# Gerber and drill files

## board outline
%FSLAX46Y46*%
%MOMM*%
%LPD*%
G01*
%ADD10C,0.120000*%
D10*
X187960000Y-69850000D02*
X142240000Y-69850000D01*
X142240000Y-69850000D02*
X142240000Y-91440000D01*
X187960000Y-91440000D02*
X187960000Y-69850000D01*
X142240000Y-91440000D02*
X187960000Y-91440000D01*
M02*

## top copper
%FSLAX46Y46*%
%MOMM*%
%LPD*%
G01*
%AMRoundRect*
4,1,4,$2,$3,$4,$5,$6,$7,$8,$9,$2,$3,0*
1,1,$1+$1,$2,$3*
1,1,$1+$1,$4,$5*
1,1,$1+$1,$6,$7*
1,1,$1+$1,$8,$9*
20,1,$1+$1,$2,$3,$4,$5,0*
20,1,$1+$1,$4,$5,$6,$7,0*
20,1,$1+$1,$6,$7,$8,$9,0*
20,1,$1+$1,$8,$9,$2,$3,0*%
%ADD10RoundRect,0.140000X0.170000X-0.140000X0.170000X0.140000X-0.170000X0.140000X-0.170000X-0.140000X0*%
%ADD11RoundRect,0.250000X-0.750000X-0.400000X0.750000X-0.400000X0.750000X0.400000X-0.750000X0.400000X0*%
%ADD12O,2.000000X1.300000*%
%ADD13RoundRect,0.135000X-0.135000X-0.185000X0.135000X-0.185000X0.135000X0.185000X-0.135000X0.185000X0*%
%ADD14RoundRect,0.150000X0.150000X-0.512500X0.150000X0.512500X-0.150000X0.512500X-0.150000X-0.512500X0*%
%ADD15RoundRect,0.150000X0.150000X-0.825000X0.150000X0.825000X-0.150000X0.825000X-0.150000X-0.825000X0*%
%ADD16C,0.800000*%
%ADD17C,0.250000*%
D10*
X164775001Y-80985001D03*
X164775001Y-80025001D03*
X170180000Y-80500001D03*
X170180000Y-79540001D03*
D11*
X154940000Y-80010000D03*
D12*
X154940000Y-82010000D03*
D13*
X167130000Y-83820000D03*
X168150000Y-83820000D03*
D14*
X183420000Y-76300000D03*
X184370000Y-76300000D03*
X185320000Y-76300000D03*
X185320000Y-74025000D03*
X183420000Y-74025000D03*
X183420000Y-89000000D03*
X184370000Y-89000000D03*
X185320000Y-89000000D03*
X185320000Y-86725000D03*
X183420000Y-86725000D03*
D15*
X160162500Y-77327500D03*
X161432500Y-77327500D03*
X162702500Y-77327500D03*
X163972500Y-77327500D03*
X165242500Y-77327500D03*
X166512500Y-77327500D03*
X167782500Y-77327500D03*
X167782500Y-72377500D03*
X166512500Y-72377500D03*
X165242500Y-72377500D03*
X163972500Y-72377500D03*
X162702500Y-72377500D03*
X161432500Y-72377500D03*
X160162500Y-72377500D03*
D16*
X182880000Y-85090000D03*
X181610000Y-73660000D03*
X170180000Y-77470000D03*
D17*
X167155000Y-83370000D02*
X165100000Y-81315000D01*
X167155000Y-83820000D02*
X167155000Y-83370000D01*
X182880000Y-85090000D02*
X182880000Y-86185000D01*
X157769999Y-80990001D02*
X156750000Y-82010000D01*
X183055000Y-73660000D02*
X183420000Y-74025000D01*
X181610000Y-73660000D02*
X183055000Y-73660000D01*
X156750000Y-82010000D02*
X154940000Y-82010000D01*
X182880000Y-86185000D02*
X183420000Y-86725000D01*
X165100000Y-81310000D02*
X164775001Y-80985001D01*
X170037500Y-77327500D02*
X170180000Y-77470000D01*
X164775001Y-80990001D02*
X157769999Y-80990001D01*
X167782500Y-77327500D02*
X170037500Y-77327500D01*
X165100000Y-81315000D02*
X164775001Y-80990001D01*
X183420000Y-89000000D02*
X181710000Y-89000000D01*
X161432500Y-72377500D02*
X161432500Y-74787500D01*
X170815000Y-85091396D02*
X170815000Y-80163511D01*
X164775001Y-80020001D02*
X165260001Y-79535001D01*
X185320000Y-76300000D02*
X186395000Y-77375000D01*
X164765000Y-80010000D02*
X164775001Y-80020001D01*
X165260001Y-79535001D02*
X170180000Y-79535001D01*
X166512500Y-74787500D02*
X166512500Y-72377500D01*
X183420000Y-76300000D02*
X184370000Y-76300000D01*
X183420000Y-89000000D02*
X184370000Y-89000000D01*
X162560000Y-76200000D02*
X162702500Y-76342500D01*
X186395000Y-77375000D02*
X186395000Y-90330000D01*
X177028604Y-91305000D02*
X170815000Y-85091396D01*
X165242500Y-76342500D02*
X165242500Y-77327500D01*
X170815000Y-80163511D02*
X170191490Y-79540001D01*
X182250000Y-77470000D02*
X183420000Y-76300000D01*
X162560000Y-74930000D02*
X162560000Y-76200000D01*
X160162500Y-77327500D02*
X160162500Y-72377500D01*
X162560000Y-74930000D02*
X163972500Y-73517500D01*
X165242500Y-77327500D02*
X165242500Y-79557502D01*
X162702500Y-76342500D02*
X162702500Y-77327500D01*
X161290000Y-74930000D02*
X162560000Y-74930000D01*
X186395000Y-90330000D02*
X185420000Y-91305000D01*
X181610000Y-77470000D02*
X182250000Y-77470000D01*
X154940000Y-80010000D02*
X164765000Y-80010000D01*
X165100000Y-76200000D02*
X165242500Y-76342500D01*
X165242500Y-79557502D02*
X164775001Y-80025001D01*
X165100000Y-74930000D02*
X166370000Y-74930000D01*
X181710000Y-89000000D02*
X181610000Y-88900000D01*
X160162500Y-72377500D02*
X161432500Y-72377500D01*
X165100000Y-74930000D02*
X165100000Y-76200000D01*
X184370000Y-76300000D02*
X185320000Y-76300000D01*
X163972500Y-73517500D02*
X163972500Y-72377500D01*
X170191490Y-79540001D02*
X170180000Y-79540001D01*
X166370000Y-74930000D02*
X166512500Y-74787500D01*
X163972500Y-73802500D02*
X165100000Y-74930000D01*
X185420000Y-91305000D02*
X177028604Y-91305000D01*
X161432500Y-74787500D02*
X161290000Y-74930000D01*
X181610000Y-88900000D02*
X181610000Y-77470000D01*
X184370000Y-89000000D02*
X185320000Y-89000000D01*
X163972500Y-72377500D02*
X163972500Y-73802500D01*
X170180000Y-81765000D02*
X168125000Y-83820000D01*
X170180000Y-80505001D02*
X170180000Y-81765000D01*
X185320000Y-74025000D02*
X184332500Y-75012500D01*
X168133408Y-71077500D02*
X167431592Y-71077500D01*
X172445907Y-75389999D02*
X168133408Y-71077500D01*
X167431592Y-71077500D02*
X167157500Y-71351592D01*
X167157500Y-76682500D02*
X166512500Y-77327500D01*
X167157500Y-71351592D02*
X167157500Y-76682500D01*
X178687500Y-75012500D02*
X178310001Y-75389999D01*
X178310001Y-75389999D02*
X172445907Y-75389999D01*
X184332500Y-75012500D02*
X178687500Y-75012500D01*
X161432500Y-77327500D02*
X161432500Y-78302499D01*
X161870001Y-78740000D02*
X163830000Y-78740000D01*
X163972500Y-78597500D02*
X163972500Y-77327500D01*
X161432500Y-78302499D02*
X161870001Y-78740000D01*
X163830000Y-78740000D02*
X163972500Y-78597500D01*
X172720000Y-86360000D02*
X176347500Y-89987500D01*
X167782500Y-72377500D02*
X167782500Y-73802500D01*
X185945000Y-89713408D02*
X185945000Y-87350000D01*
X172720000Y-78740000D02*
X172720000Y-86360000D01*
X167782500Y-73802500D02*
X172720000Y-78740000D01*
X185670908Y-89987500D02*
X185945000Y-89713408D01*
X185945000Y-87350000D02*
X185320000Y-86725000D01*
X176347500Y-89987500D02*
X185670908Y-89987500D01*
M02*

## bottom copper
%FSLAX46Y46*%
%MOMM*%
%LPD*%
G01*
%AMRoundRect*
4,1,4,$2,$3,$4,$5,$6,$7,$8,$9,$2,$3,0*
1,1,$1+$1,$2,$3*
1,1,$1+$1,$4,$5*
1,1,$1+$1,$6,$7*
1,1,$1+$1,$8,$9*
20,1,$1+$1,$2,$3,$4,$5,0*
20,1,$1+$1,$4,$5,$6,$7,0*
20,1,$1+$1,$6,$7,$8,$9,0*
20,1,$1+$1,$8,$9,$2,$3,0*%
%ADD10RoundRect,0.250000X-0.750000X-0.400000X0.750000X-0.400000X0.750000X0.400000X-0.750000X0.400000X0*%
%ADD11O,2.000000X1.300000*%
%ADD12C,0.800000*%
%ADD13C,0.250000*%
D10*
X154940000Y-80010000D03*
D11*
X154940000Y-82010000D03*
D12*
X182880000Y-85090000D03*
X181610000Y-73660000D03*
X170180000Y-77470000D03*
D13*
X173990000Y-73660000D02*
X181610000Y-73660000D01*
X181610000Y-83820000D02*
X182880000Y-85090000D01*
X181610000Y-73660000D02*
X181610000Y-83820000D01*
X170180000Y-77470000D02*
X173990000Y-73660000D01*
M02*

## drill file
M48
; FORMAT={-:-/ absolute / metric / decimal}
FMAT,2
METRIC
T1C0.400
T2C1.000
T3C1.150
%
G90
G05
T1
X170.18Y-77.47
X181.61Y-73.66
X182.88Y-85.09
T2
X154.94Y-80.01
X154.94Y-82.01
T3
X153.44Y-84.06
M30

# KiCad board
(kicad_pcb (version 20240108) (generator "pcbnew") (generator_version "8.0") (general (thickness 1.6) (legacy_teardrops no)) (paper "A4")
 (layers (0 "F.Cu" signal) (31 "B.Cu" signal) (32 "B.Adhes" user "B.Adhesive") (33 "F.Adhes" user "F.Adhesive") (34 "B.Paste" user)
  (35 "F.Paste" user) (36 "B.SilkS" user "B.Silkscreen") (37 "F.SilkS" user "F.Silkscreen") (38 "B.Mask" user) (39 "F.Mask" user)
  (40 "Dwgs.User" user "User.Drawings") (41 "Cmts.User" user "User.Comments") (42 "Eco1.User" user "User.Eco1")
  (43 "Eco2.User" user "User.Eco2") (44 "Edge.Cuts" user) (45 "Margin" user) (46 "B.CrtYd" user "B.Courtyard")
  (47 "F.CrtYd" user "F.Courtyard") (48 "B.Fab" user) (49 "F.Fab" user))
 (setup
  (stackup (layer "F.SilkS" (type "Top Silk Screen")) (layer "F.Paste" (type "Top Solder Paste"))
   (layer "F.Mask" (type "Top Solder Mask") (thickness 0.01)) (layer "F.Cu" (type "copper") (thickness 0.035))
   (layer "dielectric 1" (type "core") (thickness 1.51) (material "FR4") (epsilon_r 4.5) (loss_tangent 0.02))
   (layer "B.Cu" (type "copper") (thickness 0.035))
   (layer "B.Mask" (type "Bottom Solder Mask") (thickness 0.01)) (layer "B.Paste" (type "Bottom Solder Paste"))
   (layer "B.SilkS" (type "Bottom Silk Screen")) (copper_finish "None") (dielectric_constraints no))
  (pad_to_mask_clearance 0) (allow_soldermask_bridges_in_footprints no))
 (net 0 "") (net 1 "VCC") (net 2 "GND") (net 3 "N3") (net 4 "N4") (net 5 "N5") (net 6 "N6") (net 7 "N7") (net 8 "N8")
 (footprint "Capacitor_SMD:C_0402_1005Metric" (layer "F.Cu") (at 164.775001 80.505001 90)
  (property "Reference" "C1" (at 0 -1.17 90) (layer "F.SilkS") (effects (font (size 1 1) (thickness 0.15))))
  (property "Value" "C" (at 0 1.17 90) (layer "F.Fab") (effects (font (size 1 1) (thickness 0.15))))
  (pad "1" smd roundrect (at -0.48 0 90) (size 0.56 0.62) (layers "F.Cu" "F.Paste" "F.Mask") (roundrect_rratio 0.25) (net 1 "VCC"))
  (pad "2" smd roundrect (at 0.48 0 90) (size 0.56 0.62) (layers "F.Cu" "F.Paste" "F.Mask") (roundrect_rratio 0.25) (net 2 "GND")))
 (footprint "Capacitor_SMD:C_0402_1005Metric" (layer "F.Cu") (at 170.18 80.020001 90)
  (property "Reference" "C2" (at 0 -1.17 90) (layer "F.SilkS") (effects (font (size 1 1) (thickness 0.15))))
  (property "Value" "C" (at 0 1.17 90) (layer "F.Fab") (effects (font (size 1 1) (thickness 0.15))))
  (pad "1" smd roundrect (at -0.48 0 90) (size 0.56 0.62) (layers "F.Cu" "F.Paste" "F.Mask") (roundrect_rratio 0.25) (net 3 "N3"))
  (pad "2" smd roundrect (at 0.48 0 90) (size 0.56 0.62) (layers "F.Cu" "F.Paste" "F.Mask") (roundrect_rratio 0.25) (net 2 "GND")))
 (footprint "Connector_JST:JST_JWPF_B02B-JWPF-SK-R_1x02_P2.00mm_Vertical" (layer "F.Cu") (at 154.94 80.01)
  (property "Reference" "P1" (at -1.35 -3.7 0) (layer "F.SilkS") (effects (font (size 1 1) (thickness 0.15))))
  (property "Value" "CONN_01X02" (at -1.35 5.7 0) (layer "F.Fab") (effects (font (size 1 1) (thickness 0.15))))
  (pad "" np_thru_hole circle (at -1.5 4.05) (size 1.15 1.15) (drill 1.15) (layers "*.Cu" "*.Mask"))
  (pad "1" thru_hole roundrect (at 0 0) (size 2 1.3) (drill 1) (layers "*.Cu" "*.Mask") (remove_unused_layers no)
   (roundrect_rratio 0.192308) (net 2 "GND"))
  (pad "2" thru_hole oval (at 0 2) (size 2 1.3) (drill 1) (layers "*.Cu" "*.Mask") (remove_unused_layers no) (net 1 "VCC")))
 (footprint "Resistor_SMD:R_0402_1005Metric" (layer "F.Cu") (at 167.64 83.82)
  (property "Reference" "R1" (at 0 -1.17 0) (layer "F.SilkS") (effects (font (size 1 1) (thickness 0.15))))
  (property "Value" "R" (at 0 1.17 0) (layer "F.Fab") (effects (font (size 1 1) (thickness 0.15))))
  (pad "1" smd roundrect (at -0.51 0) (size 0.54 0.64) (layers "F.Cu" "F.Paste" "F.Mask") (roundrect_rratio 0.25) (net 1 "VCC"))
  (pad "2" smd roundrect (at 0.51 0) (size 0.54 0.64) (layers "F.Cu" "F.Paste" "F.Mask") (roundrect_rratio 0.25) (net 3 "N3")))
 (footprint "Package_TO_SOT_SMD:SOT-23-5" (layer "F.Cu") (at 184.37 75.1625 90)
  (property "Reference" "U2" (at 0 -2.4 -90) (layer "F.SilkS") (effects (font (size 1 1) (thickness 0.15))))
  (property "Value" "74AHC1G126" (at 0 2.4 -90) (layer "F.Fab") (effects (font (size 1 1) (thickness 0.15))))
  (pad "1" smd roundrect (at -1.1375 -0.95 90) (size 1.325 0.6) (layers "F.Cu" "F.Paste" "F.Mask") (roundrect_rratio 0.25) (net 2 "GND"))
  (pad "2" smd roundrect (at -1.1375 0 90) (size 1.325 0.6) (layers "F.Cu" "F.Paste" "F.Mask") (roundrect_rratio 0.25) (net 2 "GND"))
  (pad "3" smd roundrect (at -1.1375 0.95 90) (size 1.325 0.6) (layers "F.Cu" "F.Paste" "F.Mask") (roundrect_rratio 0.25) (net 2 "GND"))
  (pad "4" smd roundrect (at 1.1375 0.95 90) (size 1.325 0.6) (layers "F.Cu" "F.Paste" "F.Mask") (roundrect_rratio 0.25) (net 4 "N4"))
  (pad "5" smd roundrect (at 1.1375 -0.95 90) (size 1.325 0.6) (layers "F.Cu" "F.Paste" "F.Mask") (roundrect_rratio 0.25) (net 1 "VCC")))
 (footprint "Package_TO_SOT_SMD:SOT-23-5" (layer "F.Cu") (at 184.37 87.8625 90)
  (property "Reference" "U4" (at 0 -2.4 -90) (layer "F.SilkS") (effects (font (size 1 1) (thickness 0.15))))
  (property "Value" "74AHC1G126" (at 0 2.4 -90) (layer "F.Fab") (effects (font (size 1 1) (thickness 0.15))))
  (pad "1" smd roundrect (at -1.1375 -0.95 90) (size 1.325 0.6) (layers "F.Cu" "F.Paste" "F.Mask") (roundrect_rratio 0.25) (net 2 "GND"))
  (pad "2" smd roundrect (at -1.1375 0 90) (size 1.325 0.6) (layers "F.Cu" "F.Paste" "F.Mask") (roundrect_rratio 0.25) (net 2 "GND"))
  (pad "3" smd roundrect (at -1.1375 0.95 90) (size 1.325 0.6) (layers "F.Cu" "F.Paste" "F.Mask") (roundrect_rratio 0.25) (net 2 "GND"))
  (pad "4" smd roundrect (at 1.1375 0.95 90) (size 1.325 0.6) (layers "F.Cu" "F.Paste" "F.Mask") (roundrect_rratio 0.25) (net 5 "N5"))
  (pad "5" smd roundrect (at 1.1375 -0.95 90) (size 1.325 0.6) (layers "F.Cu" "F.Paste" "F.Mask") (roundrect_rratio 0.25) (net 1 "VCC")))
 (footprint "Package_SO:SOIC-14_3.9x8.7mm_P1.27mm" (layer "F.Cu") (at 163.9725 74.8525 90)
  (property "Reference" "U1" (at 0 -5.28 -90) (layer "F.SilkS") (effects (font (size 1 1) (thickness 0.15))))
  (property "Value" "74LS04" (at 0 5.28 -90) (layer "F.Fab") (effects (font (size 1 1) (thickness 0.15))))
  (pad "1" smd roundrect (at -2.475 -3.81 90) (size 1.95 0.6) (layers "F.Cu" "F.Paste" "F.Mask") (roundrect_rratio 0.25) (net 2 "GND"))
  (pad "2" smd roundrect (at -2.475 -2.54 90) (size 1.95 0.6) (layers "F.Cu" "F.Paste" "F.Mask") (roundrect_rratio 0.25) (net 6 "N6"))
  (pad "3" smd roundrect (at -2.475 -1.27 90) (size 1.95 0.6) (layers "F.Cu" "F.Paste" "F.Mask") (roundrect_rratio 0.25) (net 2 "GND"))
  (pad "4" smd roundrect (at -2.475 0 90) (size 1.95 0.6) (layers "F.Cu" "F.Paste" "F.Mask") (roundrect_rratio 0.25) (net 6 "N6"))
  (pad "5" smd roundrect (at -2.475 1.27 90) (size 1.95 0.6) (layers "F.Cu" "F.Paste" "F.Mask") (roundrect_rratio 0.25) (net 2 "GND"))
  (pad "6" smd roundrect (at -2.475 2.54 90) (size 1.95 0.6) (layers "F.Cu" "F.Paste" "F.Mask") (roundrect_rratio 0.25) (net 4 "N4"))
  (pad "7" smd roundrect (at -2.475 3.81 90) (size 1.95 0.6) (layers "F.Cu" "F.Paste" "F.Mask") (roundrect_rratio 0.25) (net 1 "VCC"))
  (pad "8" smd roundrect (at 2.475 3.81 90) (size 1.95 0.6) (layers "F.Cu" "F.Paste" "F.Mask") (roundrect_rratio 0.25) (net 5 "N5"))
  (pad "9" smd roundrect (at 2.475 2.54 90) (size 1.95 0.6) (layers "F.Cu" "F.Paste" "F.Mask") (roundrect_rratio 0.25) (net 2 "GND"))
  (pad "10" smd roundrect (at 2.475 1.27 90) (size 1.95 0.6) (layers "F.Cu" "F.Paste" "F.Mask") (roundrect_rratio 0.25) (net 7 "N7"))
  (pad "11" smd roundrect (at 2.475 0 90) (size 1.95 0.6) (layers "F.Cu" "F.Paste" "F.Mask") (roundrect_rratio 0.25) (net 2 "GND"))
  (pad "12" smd roundrect (at 2.475 -1.27 90) (size 1.95 0.6) (layers "F.Cu" "F.Paste" "F.Mask") (roundrect_rratio 0.25) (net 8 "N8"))
  (pad "13" smd roundrect (at 2.475 -2.54 90) (size 1.95 0.6) (layers "F.Cu" "F.Paste" "F.Mask") (roundrect_rratio 0.25) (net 2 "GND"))
  (pad "14" smd roundrect (at 2.475 -3.81 90) (size 1.95 0.6) (layers "F.Cu" "F.Paste" "F.Mask") (roundrect_rratio 0.25) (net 2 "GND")))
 (gr_line (start 187.96 69.85) (end 142.24 69.85) (stroke (width 0.12) (type solid)) (layer "Edge.Cuts"))
 (gr_line (start 142.24 69.85) (end 142.24 91.44) (stroke (width 0.12) (type solid)) (layer "Edge.Cuts"))
 (gr_line (start 187.96 91.44) (end 187.96 69.85) (stroke (width 0.12) (type solid)) (layer "Edge.Cuts"))
 (gr_line (start 142.24 91.44) (end 187.96 91.44) (stroke (width 0.12) (type solid)) (layer "Edge.Cuts"))
 (segment (start 167.155 83.37) (end 165.1 81.315) (width 0.25) (layer "F.Cu") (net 1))
 (segment (start 167.155 83.82) (end 167.155 83.37) (width 0.25) (layer "F.Cu") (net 1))
 (segment (start 182.88 85.09) (end 182.88 86.185) (width 0.25) (layer "F.Cu") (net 1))
 (segment (start 157.769999 80.990001) (end 156.75 82.01) (width 0.25) (layer "F.Cu") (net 1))
 (segment (start 183.055 73.66) (end 183.42 74.025) (width 0.25) (layer "F.Cu") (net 1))
 (segment (start 181.61 73.66) (end 183.055 73.66) (width 0.25) (layer "F.Cu") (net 1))
 (segment (start 156.75 82.01) (end 154.94 82.01) (width 0.25) (layer "F.Cu") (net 1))
 (segment (start 182.88 86.185) (end 183.42 86.725) (width 0.25) (layer "F.Cu") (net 1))
 (segment (start 165.1 81.31) (end 164.775001 80.985001) (width 0.25) (layer "F.Cu") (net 1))
 (segment (start 170.0375 77.3275) (end 170.18 77.47) (width 0.25) (layer "F.Cu") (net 1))
 (segment (start 164.775001 80.990001) (end 157.769999 80.990001) (width 0.25) (layer "F.Cu") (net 1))
 (segment (start 167.7825 77.3275) (end 170.0375 77.3275) (width 0.25) (layer "F.Cu") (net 1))
 (segment (start 165.1 81.315) (end 164.775001 80.990001) (width 0.25) (layer "F.Cu") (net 1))
 (via (at 182.88 85.09) (size 0.8) (drill 0.4) (layers "F.Cu" "B.Cu") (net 1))
 (via (at 181.61 73.66) (size 0.8) (drill 0.4) (layers "F.Cu" "B.Cu") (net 1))
 (via (at 170.18 77.47) (size 0.8) (drill 0.4) (layers "F.Cu" "B.Cu") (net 1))
 (segment (start 173.99 73.66) (end 181.61 73.66) (width 0.25) (layer "B.Cu") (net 1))
 (segment (start 181.61 83.82) (end 182.88 85.09) (width 0.25) (layer "B.Cu") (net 1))
 (segment (start 181.61 73.66) (end 181.61 83.82) (width 0.25) (layer "B.Cu") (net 1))
 (segment (start 170.18 77.47) (end 173.99 73.66) (width 0.25) (layer "B.Cu") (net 1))
 (segment (start 183.42 89) (end 181.71 89) (width 0.25) (layer "F.Cu") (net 2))
 (segment (start 161.4325 72.3775) (end 161.4325 74.7875) (width 0.25) (layer "F.Cu") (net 2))
 (segment (start 170.815 85.091396) (end 170.815 80.163511) (width 0.25) (layer "F.Cu") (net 2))
 (segment (start 164.775001 80.020001) (end 165.260001 79.535001) (width 0.25) (layer "F.Cu") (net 2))
 (segment (start 185.32 76.3) (end 186.395 77.375) (width 0.25) (layer "F.Cu") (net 2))
 (segment (start 164.765 80.01) (end 164.775001 80.020001) (width 0.25) (layer "F.Cu") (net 2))
 (segment (start 165.260001 79.535001) (end 170.18 79.535001) (width 0.25) (layer "F.Cu") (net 2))
 (segment (start 166.5125 74.7875) (end 166.5125 72.3775) (width 0.25) (layer "F.Cu") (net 2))
 (segment (start 183.42 76.3) (end 184.37 76.3) (width 0.25) (layer "F.Cu") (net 2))
 (segment (start 183.42 89) (end 184.37 89) (width 0.25) (layer "F.Cu") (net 2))
 (segment (start 162.56 76.2) (end 162.7025 76.3425) (width 0.25) (layer "F.Cu") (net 2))
 (segment (start 186.395 77.375) (end 186.395 90.33) (width 0.25) (layer "F.Cu") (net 2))
 (segment (start 177.028604 91.305) (end 170.815 85.091396) (width 0.25) (layer "F.Cu") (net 2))
 (segment (start 165.2425 76.3425) (end 165.2425 77.3275) (width 0.25) (layer "F.Cu") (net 2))
 (segment (start 170.815 80.163511) (end 170.19149 79.540001) (width 0.25) (layer "F.Cu") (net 2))
 (segment (start 182.25 77.47) (end 183.42 76.3) (width 0.25) (layer "F.Cu") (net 2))
 (segment (start 162.56 74.93) (end 162.56 76.2) (width 0.25) (layer "F.Cu") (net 2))
 (segment (start 160.1625 77.3275) (end 160.1625 72.3775) (width 0.25) (layer "F.Cu") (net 2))
 (segment (start 162.56 74.93) (end 163.9725 73.5175) (width 0.25) (layer "F.Cu") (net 2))
 (segment (start 165.2425 77.3275) (end 165.2425 79.557502) (width 0.25) (layer "F.Cu") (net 2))
 (segment (start 162.7025 76.3425) (end 162.7025 77.3275) (width 0.25) (layer "F.Cu") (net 2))
 (segment (start 161.29 74.93) (end 162.56 74.93) (width 0.25) (layer "F.Cu") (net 2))
 (segment (start 186.395 90.33) (end 185.42 91.305) (width 0.25) (layer "F.Cu") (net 2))
 (segment (start 181.61 77.47) (end 182.25 77.47) (width 0.25) (layer "F.Cu") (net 2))
 (segment (start 154.94 80.01) (end 164.765 80.01) (width 0.25) (layer "F.Cu") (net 2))
 (segment (start 165.1 76.2) (end 165.2425 76.3425) (width 0.25) (layer "F.Cu") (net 2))
 (segment (start 165.2425 79.557502) (end 164.775001 80.025001) (width 0.25) (layer "F.Cu") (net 2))
 (segment (start 165.1 74.93) (end 166.37 74.93) (width 0.25) (layer "F.Cu") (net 2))
 (segment (start 181.71 89) (end 181.61 88.9) (width 0.25) (layer "F.Cu") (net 2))
 (segment (start 160.1625 72.3775) (end 161.4325 72.3775) (width 0.25) (layer "F.Cu") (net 2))
 (segment (start 165.1 74.93) (end 165.1 76.2) (width 0.25) (layer "F.Cu") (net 2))
 (segment (start 184.37 76.3) (end 185.32 76.3) (width 0.25) (layer "F.Cu") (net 2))
 (segment (start 163.9725 73.5175) (end 163.9725 72.3775) (width 0.25) (layer "F.Cu") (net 2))
 (segment (start 170.19149 79.540001) (end 170.18 79.540001) (width 0.25) (layer "F.Cu") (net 2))
 (segment (start 166.37 74.93) (end 166.5125 74.7875) (width 0.25) (layer "F.Cu") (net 2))
 (segment (start 163.9725 73.8025) (end 165.1 74.93) (width 0.25) (layer "F.Cu") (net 2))
 (segment (start 185.42 91.305) (end 177.028604 91.305) (width 0.25) (layer "F.Cu") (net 2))
 (segment (start 161.4325 74.7875) (end 161.29 74.93) (width 0.25) (layer "F.Cu") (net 2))
 (segment (start 181.61 88.9) (end 181.61 77.47) (width 0.25) (layer "F.Cu") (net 2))
 (segment (start 184.37 89) (end 185.32 89) (width 0.25) (layer "F.Cu") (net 2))
 (segment (start 163.9725 72.3775) (end 163.9725 73.8025) (width 0.25) (layer "F.Cu") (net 2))
 (segment (start 170.18 81.765) (end 168.125 83.82) (width 0.25) (layer "F.Cu") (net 3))
 (segment (start 170.18 80.505001) (end 170.18 81.765) (width 0.25) (layer "F.Cu") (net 3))
 (segment (start 185.32 74.025) (end 184.3325 75.0125) (width 0.25) (layer "F.Cu") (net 4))
 (segment (start 168.133408 71.0775) (end 167.431592 71.0775) (width 0.25) (layer "F.Cu") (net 4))
 (segment (start 172.445907 75.389999) (end 168.133408 71.0775) (width 0.25) (layer "F.Cu") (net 4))
 (segment (start 167.431592 71.0775) (end 167.1575 71.351592) (width 0.25) (layer "F.Cu") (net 4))
 (segment (start 167.1575 76.6825) (end 166.5125 77.3275) (width 0.25) (layer "F.Cu") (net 4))
 (segment (start 167.1575 71.351592) (end 167.1575 76.6825) (width 0.25) (layer "F.Cu") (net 4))
 (segment (start 178.6875 75.0125) (end 178.310001 75.389999) (width 0.25) (layer "F.Cu") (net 4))
 (segment (start 178.310001 75.389999) (end 172.445907 75.389999) (width 0.25) (layer "F.Cu") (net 4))
 (segment (start 184.3325 75.0125) (end 178.6875 75.0125) (width 0.25) (layer "F.Cu") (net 4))
 (segment (start 161.4325 77.3275) (end 161.4325 78.302499) (width 0.25) (layer "F.Cu") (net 6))
 (segment (start 161.870001 78.74) (end 163.83 78.74) (width 0.25) (layer "F.Cu") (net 6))
 (segment (start 163.9725 78.5975) (end 163.9725 77.3275) (width 0.25) (layer "F.Cu") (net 6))
 (segment (start 161.4325 78.302499) (end 161.870001 78.74) (width 0.25) (layer "F.Cu") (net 6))
 (segment (start 163.83 78.74) (end 163.9725 78.5975) (width 0.25) (layer "F.Cu") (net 6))
 (segment (start 172.72 86.36) (end 176.3475 89.9875) (width 0.25) (layer "F.Cu") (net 5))
 (segment (start 167.7825 72.3775) (end 167.7825 73.8025) (width 0.25) (layer "F.Cu") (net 5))
 (segment (start 185.945 89.713408) (end 185.945 87.35) (width 0.25) (layer "F.Cu") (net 5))
 (segment (start 172.72 78.74) (end 172.72 86.36) (width 0.25) (layer "F.Cu") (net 5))
 (segment (start 167.7825 73.8025) (end 172.72 78.74) (width 0.25) (layer "F.Cu") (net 5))
 (segment (start 185.670908 89.9875) (end 185.945 89.713408) (width 0.25) (layer "F.Cu") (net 5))
 (segment (start 185.945 87.35) (end 185.32 86.725) (width 0.25) (layer "F.Cu") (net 5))
 (segment (start 176.3475 89.9875) (end 185.670908 89.9875) (width 0.25) (layer "F.Cu") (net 5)))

